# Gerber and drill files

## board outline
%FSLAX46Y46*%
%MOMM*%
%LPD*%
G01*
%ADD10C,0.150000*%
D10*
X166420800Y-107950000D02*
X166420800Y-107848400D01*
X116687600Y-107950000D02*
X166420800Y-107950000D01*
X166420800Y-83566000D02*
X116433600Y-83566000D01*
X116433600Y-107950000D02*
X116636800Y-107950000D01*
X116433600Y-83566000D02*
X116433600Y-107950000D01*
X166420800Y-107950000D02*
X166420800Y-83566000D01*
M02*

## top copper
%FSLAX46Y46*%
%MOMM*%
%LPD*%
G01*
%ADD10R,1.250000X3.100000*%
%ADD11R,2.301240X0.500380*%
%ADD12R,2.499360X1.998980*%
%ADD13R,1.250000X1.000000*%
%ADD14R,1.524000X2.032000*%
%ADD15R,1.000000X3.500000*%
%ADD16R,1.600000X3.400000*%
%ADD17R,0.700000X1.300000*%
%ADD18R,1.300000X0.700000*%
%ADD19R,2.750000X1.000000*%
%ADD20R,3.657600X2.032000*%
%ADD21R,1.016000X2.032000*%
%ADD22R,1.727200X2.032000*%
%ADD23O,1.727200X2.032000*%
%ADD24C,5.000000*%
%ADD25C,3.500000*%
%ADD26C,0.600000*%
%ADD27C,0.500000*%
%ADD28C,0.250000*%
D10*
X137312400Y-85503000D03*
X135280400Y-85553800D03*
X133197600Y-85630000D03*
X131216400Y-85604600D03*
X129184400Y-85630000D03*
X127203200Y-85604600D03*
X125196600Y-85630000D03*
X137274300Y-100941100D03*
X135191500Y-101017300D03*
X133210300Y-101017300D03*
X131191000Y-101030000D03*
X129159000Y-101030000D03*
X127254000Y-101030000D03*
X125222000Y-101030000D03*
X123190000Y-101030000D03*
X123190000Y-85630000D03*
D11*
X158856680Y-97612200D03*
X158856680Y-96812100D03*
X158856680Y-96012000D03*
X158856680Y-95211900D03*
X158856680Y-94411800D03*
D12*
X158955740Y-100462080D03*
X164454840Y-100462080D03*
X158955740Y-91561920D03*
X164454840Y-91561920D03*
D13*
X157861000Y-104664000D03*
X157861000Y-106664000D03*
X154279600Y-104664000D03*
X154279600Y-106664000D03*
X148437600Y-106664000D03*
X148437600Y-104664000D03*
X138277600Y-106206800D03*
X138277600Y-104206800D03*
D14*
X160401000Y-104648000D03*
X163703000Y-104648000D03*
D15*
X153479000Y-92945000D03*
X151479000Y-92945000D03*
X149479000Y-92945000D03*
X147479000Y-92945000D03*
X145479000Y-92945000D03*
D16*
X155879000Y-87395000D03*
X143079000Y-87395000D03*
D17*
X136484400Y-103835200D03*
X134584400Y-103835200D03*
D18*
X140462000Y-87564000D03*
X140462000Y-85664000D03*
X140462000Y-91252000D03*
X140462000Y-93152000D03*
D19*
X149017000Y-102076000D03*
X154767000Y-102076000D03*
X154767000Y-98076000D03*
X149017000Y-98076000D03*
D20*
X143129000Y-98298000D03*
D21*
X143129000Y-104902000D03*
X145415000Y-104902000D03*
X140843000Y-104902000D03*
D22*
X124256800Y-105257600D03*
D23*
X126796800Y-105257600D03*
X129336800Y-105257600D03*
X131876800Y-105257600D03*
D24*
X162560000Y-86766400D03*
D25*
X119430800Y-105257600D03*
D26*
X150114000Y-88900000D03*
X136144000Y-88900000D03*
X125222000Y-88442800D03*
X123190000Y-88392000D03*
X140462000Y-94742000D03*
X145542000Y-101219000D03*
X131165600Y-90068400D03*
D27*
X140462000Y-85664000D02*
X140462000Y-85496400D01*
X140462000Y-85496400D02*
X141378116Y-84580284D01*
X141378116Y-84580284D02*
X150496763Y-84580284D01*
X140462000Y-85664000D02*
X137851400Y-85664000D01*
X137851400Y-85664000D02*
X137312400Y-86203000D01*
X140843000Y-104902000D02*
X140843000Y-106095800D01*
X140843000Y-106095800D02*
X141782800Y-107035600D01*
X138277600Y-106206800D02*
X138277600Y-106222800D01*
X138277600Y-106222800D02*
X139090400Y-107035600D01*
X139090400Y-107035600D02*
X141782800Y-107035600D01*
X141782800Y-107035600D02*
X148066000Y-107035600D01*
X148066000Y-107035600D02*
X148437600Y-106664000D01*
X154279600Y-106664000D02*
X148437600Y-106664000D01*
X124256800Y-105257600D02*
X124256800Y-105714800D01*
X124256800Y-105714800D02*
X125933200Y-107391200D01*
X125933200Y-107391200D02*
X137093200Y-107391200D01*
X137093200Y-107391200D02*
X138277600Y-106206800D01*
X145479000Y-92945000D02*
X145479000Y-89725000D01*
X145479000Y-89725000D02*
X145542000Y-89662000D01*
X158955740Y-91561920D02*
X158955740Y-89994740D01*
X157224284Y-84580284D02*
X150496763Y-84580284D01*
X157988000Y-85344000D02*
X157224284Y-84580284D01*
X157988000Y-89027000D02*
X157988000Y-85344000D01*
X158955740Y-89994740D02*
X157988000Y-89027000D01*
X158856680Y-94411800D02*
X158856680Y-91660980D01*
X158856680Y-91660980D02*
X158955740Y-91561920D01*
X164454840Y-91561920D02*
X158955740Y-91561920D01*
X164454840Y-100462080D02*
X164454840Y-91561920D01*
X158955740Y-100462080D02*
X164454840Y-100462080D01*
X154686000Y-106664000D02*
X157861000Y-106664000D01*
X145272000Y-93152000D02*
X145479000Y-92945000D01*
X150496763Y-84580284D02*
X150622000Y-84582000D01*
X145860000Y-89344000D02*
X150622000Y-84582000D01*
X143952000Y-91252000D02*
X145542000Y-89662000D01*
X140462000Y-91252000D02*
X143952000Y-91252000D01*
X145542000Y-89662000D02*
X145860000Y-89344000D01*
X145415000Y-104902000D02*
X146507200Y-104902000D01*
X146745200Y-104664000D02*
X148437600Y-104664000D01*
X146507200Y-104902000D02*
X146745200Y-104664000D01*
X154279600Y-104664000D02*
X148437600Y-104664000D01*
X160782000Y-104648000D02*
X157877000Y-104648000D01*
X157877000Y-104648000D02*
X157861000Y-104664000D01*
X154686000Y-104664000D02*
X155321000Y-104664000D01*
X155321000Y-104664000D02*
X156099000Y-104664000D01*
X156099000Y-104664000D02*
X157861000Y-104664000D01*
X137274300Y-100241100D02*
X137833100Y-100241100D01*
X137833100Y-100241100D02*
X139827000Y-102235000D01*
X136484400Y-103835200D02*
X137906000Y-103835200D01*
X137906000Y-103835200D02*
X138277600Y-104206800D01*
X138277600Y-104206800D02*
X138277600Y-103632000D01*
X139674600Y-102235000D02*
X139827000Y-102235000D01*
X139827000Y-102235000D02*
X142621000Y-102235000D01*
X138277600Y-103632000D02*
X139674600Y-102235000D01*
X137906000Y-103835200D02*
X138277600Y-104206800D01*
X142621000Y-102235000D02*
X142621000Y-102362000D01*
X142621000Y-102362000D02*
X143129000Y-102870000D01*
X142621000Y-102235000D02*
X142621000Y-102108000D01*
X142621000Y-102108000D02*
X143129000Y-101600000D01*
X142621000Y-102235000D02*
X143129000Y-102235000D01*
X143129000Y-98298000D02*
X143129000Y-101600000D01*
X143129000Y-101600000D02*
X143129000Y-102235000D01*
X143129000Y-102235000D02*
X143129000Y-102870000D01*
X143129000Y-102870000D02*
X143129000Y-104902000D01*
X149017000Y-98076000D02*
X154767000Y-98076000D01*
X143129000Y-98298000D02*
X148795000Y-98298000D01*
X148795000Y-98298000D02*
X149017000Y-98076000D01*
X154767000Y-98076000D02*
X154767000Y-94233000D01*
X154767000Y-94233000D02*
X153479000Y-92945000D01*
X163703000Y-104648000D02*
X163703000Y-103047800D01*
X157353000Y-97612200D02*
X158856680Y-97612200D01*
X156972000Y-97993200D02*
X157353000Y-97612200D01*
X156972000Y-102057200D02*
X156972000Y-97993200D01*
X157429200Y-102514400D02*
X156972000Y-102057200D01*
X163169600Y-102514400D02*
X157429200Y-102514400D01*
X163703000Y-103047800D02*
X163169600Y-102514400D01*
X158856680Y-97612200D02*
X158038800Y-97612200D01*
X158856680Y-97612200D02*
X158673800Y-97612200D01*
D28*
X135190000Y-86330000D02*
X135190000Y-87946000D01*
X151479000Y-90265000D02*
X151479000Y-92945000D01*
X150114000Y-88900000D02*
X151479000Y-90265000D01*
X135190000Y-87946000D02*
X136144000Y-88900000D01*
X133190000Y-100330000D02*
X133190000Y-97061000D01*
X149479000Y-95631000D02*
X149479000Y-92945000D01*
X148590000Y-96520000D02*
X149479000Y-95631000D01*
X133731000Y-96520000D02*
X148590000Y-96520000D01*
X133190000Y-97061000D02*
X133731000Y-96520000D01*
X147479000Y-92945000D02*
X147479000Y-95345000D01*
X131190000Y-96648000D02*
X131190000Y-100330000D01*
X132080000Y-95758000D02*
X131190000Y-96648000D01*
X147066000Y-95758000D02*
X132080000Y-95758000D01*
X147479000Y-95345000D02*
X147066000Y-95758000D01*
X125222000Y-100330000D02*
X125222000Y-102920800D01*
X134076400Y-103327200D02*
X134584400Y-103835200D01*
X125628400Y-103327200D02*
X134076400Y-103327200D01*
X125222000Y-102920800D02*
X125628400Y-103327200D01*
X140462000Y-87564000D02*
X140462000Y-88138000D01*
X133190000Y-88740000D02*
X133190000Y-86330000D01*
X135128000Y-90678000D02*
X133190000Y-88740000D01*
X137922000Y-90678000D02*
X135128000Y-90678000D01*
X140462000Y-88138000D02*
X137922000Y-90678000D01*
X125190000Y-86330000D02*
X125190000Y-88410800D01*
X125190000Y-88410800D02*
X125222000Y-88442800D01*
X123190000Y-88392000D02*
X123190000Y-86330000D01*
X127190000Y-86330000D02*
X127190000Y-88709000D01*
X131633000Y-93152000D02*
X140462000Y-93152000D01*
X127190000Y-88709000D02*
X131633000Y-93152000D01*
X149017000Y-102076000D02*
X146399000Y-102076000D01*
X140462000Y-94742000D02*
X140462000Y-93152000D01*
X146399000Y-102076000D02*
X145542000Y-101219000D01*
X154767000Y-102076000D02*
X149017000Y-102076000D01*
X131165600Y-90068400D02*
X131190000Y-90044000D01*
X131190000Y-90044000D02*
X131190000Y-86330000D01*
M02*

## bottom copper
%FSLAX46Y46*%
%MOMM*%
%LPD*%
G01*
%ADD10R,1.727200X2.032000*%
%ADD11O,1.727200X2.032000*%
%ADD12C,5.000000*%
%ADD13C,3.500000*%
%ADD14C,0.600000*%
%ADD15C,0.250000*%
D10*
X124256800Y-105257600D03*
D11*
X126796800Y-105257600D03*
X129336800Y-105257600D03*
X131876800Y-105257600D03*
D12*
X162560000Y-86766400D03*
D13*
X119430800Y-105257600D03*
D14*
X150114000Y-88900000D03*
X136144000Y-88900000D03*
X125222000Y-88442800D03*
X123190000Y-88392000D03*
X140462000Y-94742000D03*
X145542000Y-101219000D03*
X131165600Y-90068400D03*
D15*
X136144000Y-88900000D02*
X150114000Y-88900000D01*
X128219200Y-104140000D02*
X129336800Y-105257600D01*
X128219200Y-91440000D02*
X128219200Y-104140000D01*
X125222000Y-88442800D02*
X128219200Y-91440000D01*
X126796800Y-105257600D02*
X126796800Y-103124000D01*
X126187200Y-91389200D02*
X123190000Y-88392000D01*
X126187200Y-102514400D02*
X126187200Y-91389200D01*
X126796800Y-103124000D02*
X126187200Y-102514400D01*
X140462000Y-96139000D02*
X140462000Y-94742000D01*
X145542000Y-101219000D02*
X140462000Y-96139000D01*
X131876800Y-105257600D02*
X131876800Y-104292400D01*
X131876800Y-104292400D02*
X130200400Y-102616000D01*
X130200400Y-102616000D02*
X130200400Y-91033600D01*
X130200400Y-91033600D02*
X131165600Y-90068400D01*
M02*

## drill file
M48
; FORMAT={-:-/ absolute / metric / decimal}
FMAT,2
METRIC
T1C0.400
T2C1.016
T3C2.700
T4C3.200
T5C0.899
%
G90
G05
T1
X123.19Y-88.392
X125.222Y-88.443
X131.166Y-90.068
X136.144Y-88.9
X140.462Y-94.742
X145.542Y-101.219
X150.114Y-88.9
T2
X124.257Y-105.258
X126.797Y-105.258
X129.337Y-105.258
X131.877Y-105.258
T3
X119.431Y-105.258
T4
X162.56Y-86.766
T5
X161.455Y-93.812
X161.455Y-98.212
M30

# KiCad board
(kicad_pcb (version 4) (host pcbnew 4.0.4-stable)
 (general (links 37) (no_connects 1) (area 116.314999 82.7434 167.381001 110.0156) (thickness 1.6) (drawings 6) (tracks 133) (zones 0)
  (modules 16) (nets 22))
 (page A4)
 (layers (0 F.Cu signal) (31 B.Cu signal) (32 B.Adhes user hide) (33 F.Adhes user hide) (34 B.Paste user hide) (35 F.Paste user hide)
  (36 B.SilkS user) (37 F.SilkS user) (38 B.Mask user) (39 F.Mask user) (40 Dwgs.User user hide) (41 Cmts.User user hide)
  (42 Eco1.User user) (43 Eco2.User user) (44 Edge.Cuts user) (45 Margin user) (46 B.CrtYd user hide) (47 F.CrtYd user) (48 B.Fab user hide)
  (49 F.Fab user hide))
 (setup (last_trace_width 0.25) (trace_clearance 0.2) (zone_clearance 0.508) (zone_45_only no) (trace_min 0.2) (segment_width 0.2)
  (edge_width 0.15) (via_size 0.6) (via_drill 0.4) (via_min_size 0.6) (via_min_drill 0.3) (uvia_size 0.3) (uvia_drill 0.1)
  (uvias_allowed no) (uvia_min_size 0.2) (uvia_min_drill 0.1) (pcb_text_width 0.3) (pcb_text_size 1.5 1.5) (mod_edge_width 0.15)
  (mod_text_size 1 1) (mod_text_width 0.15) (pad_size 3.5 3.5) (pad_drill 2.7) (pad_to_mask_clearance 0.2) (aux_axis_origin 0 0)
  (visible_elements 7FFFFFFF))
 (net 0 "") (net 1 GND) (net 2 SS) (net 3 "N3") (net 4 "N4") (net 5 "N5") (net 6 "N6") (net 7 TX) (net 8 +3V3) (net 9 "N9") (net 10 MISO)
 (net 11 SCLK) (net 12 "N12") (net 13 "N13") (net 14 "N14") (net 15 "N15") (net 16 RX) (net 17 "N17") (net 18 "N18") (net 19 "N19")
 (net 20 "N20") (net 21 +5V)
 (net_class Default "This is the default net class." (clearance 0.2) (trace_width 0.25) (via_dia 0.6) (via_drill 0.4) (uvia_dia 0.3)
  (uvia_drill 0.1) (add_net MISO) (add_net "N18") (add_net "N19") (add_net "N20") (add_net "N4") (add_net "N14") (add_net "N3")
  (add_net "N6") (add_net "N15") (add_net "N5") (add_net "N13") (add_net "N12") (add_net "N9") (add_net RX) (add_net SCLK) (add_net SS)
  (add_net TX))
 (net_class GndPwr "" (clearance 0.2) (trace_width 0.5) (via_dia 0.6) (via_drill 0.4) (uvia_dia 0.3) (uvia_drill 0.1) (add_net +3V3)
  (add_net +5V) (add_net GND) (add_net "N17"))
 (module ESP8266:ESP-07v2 (layer F.Cu) (at 123.19 100.33 90)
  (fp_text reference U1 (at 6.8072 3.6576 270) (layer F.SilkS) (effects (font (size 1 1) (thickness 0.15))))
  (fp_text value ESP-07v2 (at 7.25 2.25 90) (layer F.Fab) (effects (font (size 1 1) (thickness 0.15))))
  (pad 9 smd rect (at 14.127 14.1224 90) (size 3.1 1.25) (drill (offset 0.7 0)) (layers F.Cu F.Paste F.Mask) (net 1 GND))
  (pad 10 smd rect (at 14.0762 12.0904 90) (size 3.1 1.25) (drill (offset 0.7 0)) (layers F.Cu F.Paste F.Mask) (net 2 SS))
  (pad 11 smd rect (at 14 10.0076 90) (size 3.1 1.25) (drill (offset 0.7 0)) (layers F.Cu F.Paste F.Mask) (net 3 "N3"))
  (pad 12 smd rect (at 14.0254 8.0264 90) (size 3.1 1.25) (drill (offset 0.7 0)) (layers F.Cu F.Paste F.Mask) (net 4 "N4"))
  (pad 13 smd rect (at 14 5.9944 90) (size 3.1 1.25) (drill (offset 0.7 0)) (layers F.Cu F.Paste F.Mask) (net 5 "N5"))
  (pad 14 smd rect (at 14.0254 4.0132 90) (size 3.1 1.25) (drill (offset 0.7 0)) (layers F.Cu F.Paste F.Mask) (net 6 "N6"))
  (pad 15 smd rect (at 14 2.0066 90) (size 3.1 1.25) (drill (offset 0.7 0)) (layers F.Cu F.Paste F.Mask) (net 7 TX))
  (pad 8 smd rect (at 0.0889 14.0843 90) (size 3.1 1.25) (drill (offset -0.7 0)) (layers F.Cu F.Paste F.Mask) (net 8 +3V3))
  (pad 7 smd rect (at 0.0127 12.0015 90) (size 3.1 1.25) (drill (offset -0.7 0)) (layers F.Cu F.Paste F.Mask) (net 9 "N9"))
  (pad 6 smd rect (at 0.0127 10.0203 90) (size 3.1 1.25) (drill (offset -0.7 0)) (layers F.Cu F.Paste F.Mask) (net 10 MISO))
  (pad 5 smd rect (at 0 8.001 90) (size 3.1 1.25) (drill (offset -0.7 0)) (layers F.Cu F.Paste F.Mask) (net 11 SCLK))
  (pad 4 smd rect (at 0 5.969 90) (size 3.1 1.25) (drill (offset -0.7 0)) (layers F.Cu F.Paste F.Mask) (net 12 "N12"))
  (pad 3 smd rect (at 0 4.064 90) (size 3.1 1.25) (drill (offset -0.7 0)) (layers F.Cu F.Paste F.Mask) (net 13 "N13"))
  (pad 2 smd rect (at 0 2.032 90) (size 3.1 1.25) (drill (offset -0.7 0)) (layers F.Cu F.Paste F.Mask) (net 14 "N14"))
  (pad 1 smd rect (at 0 0 90) (size 3.1 1.25) (drill (offset -0.7 0)) (layers F.Cu F.Paste F.Mask) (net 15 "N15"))
  (pad 16 smd rect (at 14 0 90) (size 3.1 1.25) (drill (offset 0.7 0)) (layers F.Cu F.Paste F.Mask) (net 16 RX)))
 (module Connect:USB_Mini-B (layer F.Cu) (at 162.306 96.012 180)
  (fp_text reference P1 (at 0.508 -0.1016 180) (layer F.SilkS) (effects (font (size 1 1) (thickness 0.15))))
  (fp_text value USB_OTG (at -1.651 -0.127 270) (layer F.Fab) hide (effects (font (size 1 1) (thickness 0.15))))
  (pad 1 smd rect (at 3.44932 -1.6002 180) (size 2.30124 0.50038) (layers F.Cu F.Paste F.Mask) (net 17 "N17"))
  (pad 2 smd rect (at 3.44932 -0.8001 180) (size 2.30124 0.50038) (layers F.Cu F.Paste F.Mask) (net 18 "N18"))
  (pad 3 smd rect (at 3.44932 0 180) (size 2.30124 0.50038) (layers F.Cu F.Paste F.Mask) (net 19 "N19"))
  (pad 4 smd rect (at 3.44932 0.8001 180) (size 2.30124 0.50038) (layers F.Cu F.Paste F.Mask) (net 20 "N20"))
  (pad 5 smd rect (at 3.44932 1.6002 180) (size 2.30124 0.50038) (layers F.Cu F.Paste F.Mask) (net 1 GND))
  (pad 6 smd rect (at 3.35026 -4.45008 180) (size 2.49936 1.99898) (layers F.Cu F.Paste F.Mask) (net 1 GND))
  (pad 6 smd rect (at -2.14884 -4.45008 180) (size 2.49936 1.99898) (layers F.Cu F.Paste F.Mask) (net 1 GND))
  (pad 6 smd rect (at 3.35026 4.45008 180) (size 2.49936 1.99898) (layers F.Cu F.Paste F.Mask) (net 1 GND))
  (pad 6 smd rect (at -2.14884 4.45008 180) (size 2.49936 1.99898) (layers F.Cu F.Paste F.Mask) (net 1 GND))
  (pad "" np_thru_hole circle (at 0.8509 -2.19964 180) (size 0.89916 0.89916) (drill 0.89916) (layers *.Cu *.Mask F.SilkS))
  (pad "" np_thru_hole circle (at 0.8509 2.19964 180) (size 0.89916 0.89916) (drill 0.89916) (layers *.Cu *.Mask F.SilkS)))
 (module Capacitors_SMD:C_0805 (layer F.Cu) (at 157.861 105.664 270)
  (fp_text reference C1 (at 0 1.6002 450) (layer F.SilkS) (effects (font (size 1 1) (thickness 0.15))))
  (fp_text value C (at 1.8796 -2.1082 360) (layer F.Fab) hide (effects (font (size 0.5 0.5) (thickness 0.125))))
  (pad 1 smd rect (at -1 0 270) (size 1 1.25) (layers F.Cu F.Paste F.Mask) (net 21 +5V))
  (pad 2 smd rect (at 1 0 270) (size 1 1.25) (layers F.Cu F.Paste F.Mask) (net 1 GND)))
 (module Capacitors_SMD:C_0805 (layer F.Cu) (at 154.2796 105.664 270)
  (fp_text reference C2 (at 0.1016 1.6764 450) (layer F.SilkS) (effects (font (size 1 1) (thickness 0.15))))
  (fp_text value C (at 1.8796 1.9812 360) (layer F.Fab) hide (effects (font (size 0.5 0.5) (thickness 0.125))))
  (pad 1 smd rect (at -1 0 270) (size 1 1.25) (layers F.Cu F.Paste F.Mask) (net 21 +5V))
  (pad 2 smd rect (at 1 0 270) (size 1 1.25) (layers F.Cu F.Paste F.Mask) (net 1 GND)))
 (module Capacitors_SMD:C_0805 (layer F.Cu) (at 148.4376 105.664 90)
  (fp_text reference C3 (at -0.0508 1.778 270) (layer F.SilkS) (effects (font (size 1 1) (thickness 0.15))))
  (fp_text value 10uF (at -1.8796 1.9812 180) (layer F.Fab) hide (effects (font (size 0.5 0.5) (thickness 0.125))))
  (pad 1 smd rect (at -1 0 90) (size 1 1.25) (layers F.Cu F.Paste F.Mask) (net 1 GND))
  (pad 2 smd rect (at 1 0 90) (size 1 1.25) (layers F.Cu F.Paste F.Mask) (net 21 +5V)))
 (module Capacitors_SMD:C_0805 (layer F.Cu) (at 138.2776 105.2068 90)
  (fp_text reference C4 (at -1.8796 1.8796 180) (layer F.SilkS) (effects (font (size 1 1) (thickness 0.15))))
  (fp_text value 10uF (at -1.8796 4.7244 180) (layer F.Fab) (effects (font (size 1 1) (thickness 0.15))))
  (pad 1 smd rect (at -1 0 90) (size 1 1.25) (layers F.Cu F.Paste F.Mask) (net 1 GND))
  (pad 2 smd rect (at 1 0 90) (size 1 1.25) (layers F.Cu F.Paste F.Mask) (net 8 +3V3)))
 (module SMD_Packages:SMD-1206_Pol (layer F.Cu) (at 162.052 104.648)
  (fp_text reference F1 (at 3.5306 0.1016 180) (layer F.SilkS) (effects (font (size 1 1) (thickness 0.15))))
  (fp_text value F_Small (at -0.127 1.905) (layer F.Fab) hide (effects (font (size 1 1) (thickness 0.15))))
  (pad 1 smd rect (at -1.651 0) (size 1.524 2.032) (layers F.Cu F.Paste F.Mask) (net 21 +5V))
  (pad 2 smd rect (at 1.651 0) (size 1.524 2.032) (layers F.Cu F.Paste F.Mask) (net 17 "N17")))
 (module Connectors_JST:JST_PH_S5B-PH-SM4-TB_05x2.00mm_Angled (layer F.Cu) (at 149.479 90.17 180)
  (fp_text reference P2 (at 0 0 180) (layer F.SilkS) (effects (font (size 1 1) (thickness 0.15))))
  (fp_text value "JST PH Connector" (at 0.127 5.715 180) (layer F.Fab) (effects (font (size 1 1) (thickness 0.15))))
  (pad 1 smd rect (at -4 -2.775 180) (size 1 3.5) (layers F.Cu F.Paste F.Mask) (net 8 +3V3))
  (pad 2 smd rect (at -2 -2.775 180) (size 1 3.5) (layers F.Cu F.Paste F.Mask) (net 2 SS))
  (pad 3 smd rect (at 0 -2.775 180) (size 1 3.5) (layers F.Cu F.Paste F.Mask) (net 10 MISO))
  (pad 4 smd rect (at 2 -2.775 180) (size 1 3.5) (layers F.Cu F.Paste F.Mask) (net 11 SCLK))
  (pad 5 smd rect (at 4 -2.775 180) (size 1 3.5) (layers F.Cu F.Paste F.Mask) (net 1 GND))
  (pad "" smd rect (at -6.4 2.775 180) (size 1.6 3.4) (layers F.Cu F.Paste F.Mask))
  (pad "" smd rect (at 6.4 2.775 180) (size 1.6 3.4) (layers F.Cu F.Paste F.Mask)))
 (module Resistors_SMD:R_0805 (layer F.Cu) (at 135.5344 103.8352 180)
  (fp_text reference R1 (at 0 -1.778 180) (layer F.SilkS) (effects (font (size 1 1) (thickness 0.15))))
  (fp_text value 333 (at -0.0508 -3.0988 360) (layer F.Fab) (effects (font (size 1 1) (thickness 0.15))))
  (pad 1 smd rect (at -0.95 0 180) (size 0.7 1.3) (layers F.Cu F.Paste F.Mask) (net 8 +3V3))
  (pad 2 smd rect (at 0.95 0 180) (size 0.7 1.3) (layers F.Cu F.Paste F.Mask) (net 14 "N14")))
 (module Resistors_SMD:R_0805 (layer F.Cu) (at 140.462 86.614 90)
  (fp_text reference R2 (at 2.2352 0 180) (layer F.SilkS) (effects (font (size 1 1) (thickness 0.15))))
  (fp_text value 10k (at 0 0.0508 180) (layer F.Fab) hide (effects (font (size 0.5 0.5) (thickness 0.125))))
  (pad 1 smd rect (at -0.95 0 90) (size 0.7 1.3) (layers F.Cu F.Paste F.Mask) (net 3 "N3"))
  (pad 2 smd rect (at 0.95 0 90) (size 0.7 1.3) (layers F.Cu F.Paste F.Mask) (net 1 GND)))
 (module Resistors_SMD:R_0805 (layer F.Cu) (at 140.462 92.202 270)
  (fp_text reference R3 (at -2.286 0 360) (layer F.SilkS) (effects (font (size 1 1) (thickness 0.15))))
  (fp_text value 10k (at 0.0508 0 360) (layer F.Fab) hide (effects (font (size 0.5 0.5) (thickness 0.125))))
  (pad 1 smd rect (at -0.95 0 270) (size 0.7 1.3) (layers F.Cu F.Paste F.Mask) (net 1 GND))
  (pad 2 smd rect (at 0.95 0 270) (size 0.7 1.3) (layers F.Cu F.Paste F.Mask) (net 6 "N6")))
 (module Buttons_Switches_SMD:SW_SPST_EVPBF (layer F.Cu) (at 151.892 100.076 180)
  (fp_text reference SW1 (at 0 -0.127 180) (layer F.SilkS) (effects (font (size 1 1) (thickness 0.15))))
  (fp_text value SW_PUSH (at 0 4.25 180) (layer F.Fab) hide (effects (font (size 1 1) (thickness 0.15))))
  (pad 1 smd rect (at 2.875 -2 180) (size 2.75 1) (layers F.Cu F.Paste F.Mask) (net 6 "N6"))
  (pad 1 smd rect (at -2.875 -2 180) (size 2.75 1) (layers F.Cu F.Paste F.Mask) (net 6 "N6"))
  (pad 2 smd rect (at -2.875 2 180) (size 2.75 1) (layers F.Cu F.Paste F.Mask) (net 8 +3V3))
  (pad 2 smd rect (at 2.875 2 180) (size 2.75 1) (layers F.Cu F.Paste F.Mask) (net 8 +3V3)))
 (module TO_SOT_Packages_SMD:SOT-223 (layer F.Cu) (at 143.129 101.6)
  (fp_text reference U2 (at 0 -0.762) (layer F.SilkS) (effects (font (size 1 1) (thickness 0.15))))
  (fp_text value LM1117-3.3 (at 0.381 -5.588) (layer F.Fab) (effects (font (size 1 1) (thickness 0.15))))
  (pad 4 smd rect (at 0 -3.302) (size 3.6576 2.032) (layers F.Cu F.Paste F.Mask) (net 8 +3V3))
  (pad 2 smd rect (at 0 3.302) (size 1.016 2.032) (layers F.Cu F.Paste F.Mask) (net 8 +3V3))
  (pad 3 smd rect (at 2.286 3.302) (size 1.016 2.032) (layers F.Cu F.Paste F.Mask) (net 21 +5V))
  (pad 1 smd rect (at -2.286 3.302) (size 1.016 2.032) (layers F.Cu F.Paste F.Mask) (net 1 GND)))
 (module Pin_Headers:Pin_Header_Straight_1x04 (layer F.Cu) (at 124.2568 105.2576 90)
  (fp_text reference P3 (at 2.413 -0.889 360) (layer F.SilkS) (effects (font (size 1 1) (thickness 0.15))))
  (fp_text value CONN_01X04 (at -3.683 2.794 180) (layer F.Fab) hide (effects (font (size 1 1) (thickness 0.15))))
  (pad 1 thru_hole rect (at 0 0 90) (size 2.032 1.7272) (drill 1.016) (layers *.Cu *.Mask F.SilkS) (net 1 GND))
  (pad 2 thru_hole oval (at 0 2.54 90) (size 2.032 1.7272) (drill 1.016) (layers *.Cu *.Mask F.SilkS) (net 16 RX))
  (pad 3 thru_hole oval (at 0 5.08 90) (size 2.032 1.7272) (drill 1.016) (layers *.Cu *.Mask F.SilkS) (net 7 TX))
  (pad 4 thru_hole oval (at 0 7.62 90) (size 2.032 1.7272) (drill 1.016) (layers *.Cu *.Mask F.SilkS) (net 4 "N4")))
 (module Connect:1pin (layer F.Cu) (at 162.56 86.7664)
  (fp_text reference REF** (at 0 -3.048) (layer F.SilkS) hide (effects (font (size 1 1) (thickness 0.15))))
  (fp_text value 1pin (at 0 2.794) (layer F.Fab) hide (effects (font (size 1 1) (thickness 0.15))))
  (pad 1 thru_hole circle (at 0 0) (size 5 5) (drill 3.2) (layers *.Cu *.Mask F.SilkS)))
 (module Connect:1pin (layer F.Cu) (at 119.4308 105.2576)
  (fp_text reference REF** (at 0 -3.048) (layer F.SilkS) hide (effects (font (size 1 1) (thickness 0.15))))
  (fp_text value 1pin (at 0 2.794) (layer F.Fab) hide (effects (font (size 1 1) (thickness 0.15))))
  (pad 1 thru_hole circle (at 0 0) (size 3.5 3.5) (drill 2.7) (layers *.Cu *.Mask F.SilkS)))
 (gr_line (start 166.4208 107.95) (end 166.4208 107.8484) (angle 90) (layer Edge.Cuts) (width 0.15))
 (gr_line (start 116.6876 107.95) (end 166.4208 107.95) (angle 90) (layer Edge.Cuts) (width 0.15))
 (gr_line (start 166.4208 83.566) (end 116.4336 83.566) (angle 90) (layer Edge.Cuts) (width 0.15))
 (gr_line (start 116.4336 107.95) (end 116.6368 107.95) (angle 90) (layer Edge.Cuts) (width 0.15))
 (gr_line (start 116.4336 83.566) (end 116.4336 107.95) (angle 90) (layer Edge.Cuts) (width 0.15))
 (gr_line (start 166.4208 107.95) (end 166.4208 83.566) (angle 90) (layer Edge.Cuts) (width 0.15))
 (segment (start 140.462 85.664) (end 140.462 85.4964) (width 0.5) (layer F.Cu) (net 1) (status C00000))
 (segment (start 140.462 85.4964) (end 141.378116 84.580284) (width 0.5) (layer F.Cu) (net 1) (status 400000))
 (segment (start 141.378116 84.580284) (end 150.496763 84.580284) (width 0.5) (layer F.Cu) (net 1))
 (segment (start 140.462 85.664) (end 137.8514 85.664) (width 0.5) (layer F.Cu) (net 1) (status C00000))
 (segment (start 137.8514 85.664) (end 137.3124 86.203) (width 0.5) (layer F.Cu) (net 1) (status C00000))
 (segment (start 140.843 104.902) (end 140.843 106.0958) (width 0.5) (layer F.Cu) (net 1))
 (segment (start 140.843 106.0958) (end 141.7828 107.0356) (width 0.5) (layer F.Cu) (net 1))
 (segment (start 138.2776 106.2068) (end 138.2776 106.2228) (width 0.5) (layer F.Cu) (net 1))
 (segment (start 138.2776 106.2228) (end 139.0904 107.0356) (width 0.5) (layer F.Cu) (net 1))
 (segment (start 139.0904 107.0356) (end 141.7828 107.0356) (width 0.5) (layer F.Cu) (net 1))
 (segment (start 141.7828 107.0356) (end 148.066 107.0356) (width 0.5) (layer F.Cu) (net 1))
 (segment (start 148.066 107.0356) (end 148.4376 106.664) (width 0.5) (layer F.Cu) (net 1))
 (segment (start 154.2796 106.664) (end 148.4376 106.664) (width 0.5) (layer F.Cu) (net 1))
 (segment (start 124.2568 105.2576) (end 124.2568 105.7148) (width 0.5) (layer F.Cu) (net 1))
 (segment (start 124.2568 105.7148) (end 125.9332 107.3912) (width 0.5) (layer F.Cu) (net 1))
 (segment (start 125.9332 107.3912) (end 137.0932 107.3912) (width 0.5) (layer F.Cu) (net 1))
 (segment (start 137.0932 107.3912) (end 138.2776 106.2068) (width 0.5) (layer F.Cu) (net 1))
 (segment (start 145.479 92.945) (end 145.479 89.725) (width 0.5) (layer F.Cu) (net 1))
 (segment (start 145.479 89.725) (end 145.542 89.662) (width 0.5) (layer F.Cu) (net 1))
 (segment (start 158.95574 91.56192) (end 158.95574 89.99474) (width 0.5) (layer F.Cu) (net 1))
 (segment (start 157.224284 84.580284) (end 150.496763 84.580284) (width 0.5) (layer F.Cu) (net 1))
 (segment (start 157.988 85.344) (end 157.224284 84.580284) (width 0.5) (layer F.Cu) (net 1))
 (segment (start 157.988 89.027) (end 157.988 85.344) (width 0.5) (layer F.Cu) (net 1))
 (segment (start 158.95574 89.99474) (end 157.988 89.027) (width 0.5) (layer F.Cu) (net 1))
 (segment (start 158.85668 94.4118) (end 158.85668 91.66098) (width 0.5) (layer F.Cu) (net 1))
 (segment (start 158.85668 91.66098) (end 158.95574 91.56192) (width 0.5) (layer F.Cu) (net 1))
 (segment (start 164.45484 91.56192) (end 158.95574 91.56192) (width 0.5) (layer F.Cu) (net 1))
 (segment (start 164.45484 100.46208) (end 164.45484 91.56192) (width 0.5) (layer F.Cu) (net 1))
 (segment (start 158.95574 100.46208) (end 164.45484 100.46208) (width 0.5) (layer F.Cu) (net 1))
 (segment (start 154.686 106.664) (end 157.861 106.664) (width 0.5) (layer F.Cu) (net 1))
 (segment (start 145.272 93.152) (end 145.479 92.945) (width 0.5) (layer F.Cu) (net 1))
 (segment (start 150.496763 84.580284) (end 150.622 84.582) (width 0.5) (layer F.Cu) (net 1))
 (segment (start 145.86 89.344) (end 150.622 84.582) (width 0.5) (layer F.Cu) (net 1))
 (segment (start 143.952 91.252) (end 145.542 89.662) (width 0.5) (layer F.Cu) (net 1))
 (segment (start 140.462 91.252) (end 143.952 91.252) (width 0.5) (layer F.Cu) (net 1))
 (segment (start 145.542 89.662) (end 145.86 89.344) (width 0.5) (layer F.Cu) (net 1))
 (segment (start 145.415 104.902) (end 146.5072 104.902) (width 0.5) (layer F.Cu) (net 21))
 (segment (start 146.7452 104.664) (end 148.4376 104.664) (width 0.5) (layer F.Cu) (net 21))
 (segment (start 146.5072 104.902) (end 146.7452 104.664) (width 0.5) (layer F.Cu) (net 21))
 (segment (start 154.2796 104.664) (end 148.4376 104.664) (width 0.5) (layer F.Cu) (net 21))
 (segment (start 160.782 104.648) (end 157.877 104.648) (width 0.5) (layer F.Cu) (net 21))
 (segment (start 157.877 104.648) (end 157.861 104.664) (width 0.5) (layer F.Cu) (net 21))
 (segment (start 154.686 104.664) (end 155.321 104.664) (width 0.5) (layer F.Cu) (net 21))
 (segment (start 155.321 104.664) (end 156.099 104.664) (width 0.5) (layer F.Cu) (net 21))
 (segment (start 156.099 104.664) (end 157.861 104.664) (width 0.5) (layer F.Cu) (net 21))
 (segment (start 137.2743 100.2411) (end 137.8331 100.2411) (width 0.5) (layer F.Cu) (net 8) (status C00000))
 (segment (start 137.8331 100.2411) (end 139.827 102.235) (width 0.5) (layer F.Cu) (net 8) (status 400000))
 (segment (start 136.4844 103.8352) (end 137.906 103.8352) (width 0.5) (layer F.Cu) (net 8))
 (segment (start 137.906 103.8352) (end 138.2776 104.2068) (width 0.5) (layer F.Cu) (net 8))
 (segment (start 138.2776 104.2068) (end 138.2776 103.632) (width 0.5) (layer F.Cu) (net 8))
 (segment (start 139.6746 102.235) (end 139.827 102.235) (width 0.5) (layer F.Cu) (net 8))
 (segment (start 139.827 102.235) (end 142.621 102.235) (width 0.5) (layer F.Cu) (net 8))
 (segment (start 138.2776 103.632) (end 139.6746 102.235) (width 0.5) (layer F.Cu) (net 8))
 (segment (start 137.906 103.8352) (end 138.2776 104.2068) (width 0.5) (layer F.Cu) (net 8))
 (segment (start 142.621 102.235) (end 142.621 102.362) (width 0.5) (layer F.Cu) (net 8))
 (segment (start 142.621 102.362) (end 143.129 102.87) (width 0.5) (layer F.Cu) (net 8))
 (segment (start 142.621 102.235) (end 142.621 102.108) (width 0.5) (layer F.Cu) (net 8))
 (segment (start 142.621 102.108) (end 143.129 101.6) (width 0.5) (layer F.Cu) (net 8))
 (segment (start 142.621 102.235) (end 143.129 102.235) (width 0.5) (layer F.Cu) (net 8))
 (segment (start 143.129 98.298) (end 143.129 101.6) (width 0.5) (layer F.Cu) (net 8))
 (segment (start 143.129 101.6) (end 143.129 102.235) (width 0.5) (layer F.Cu) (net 8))
 (segment (start 143.129 102.235) (end 143.129 102.87) (width 0.5) (layer F.Cu) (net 8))
 (segment (start 143.129 102.87) (end 143.129 104.902) (width 0.5) (layer F.Cu) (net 8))
 (segment (start 149.017 98.076) (end 154.767 98.076) (width 0.5) (layer F.Cu) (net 8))
 (segment (start 143.129 98.298) (end 148.795 98.298) (width 0.5) (layer F.Cu) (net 8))
 (segment (start 148.795 98.298) (end 149.017 98.076) (width 0.5) (layer F.Cu) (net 8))
 (segment (start 154.767 98.076) (end 154.767 94.233) (width 0.5) (layer F.Cu) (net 8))
 (segment (start 154.767 94.233) (end 153.479 92.945) (width 0.5) (layer F.Cu) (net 8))
 (segment (start 163.703 104.648) (end 163.703 103.0478) (width 0.5) (layer F.Cu) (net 17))
 (segment (start 157.353 97.6122) (end 158.85668 97.6122) (width 0.5) (layer F.Cu) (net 17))
 (segment (start 156.972 97.9932) (end 157.353 97.6122) (width 0.5) (layer F.Cu) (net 17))
 (segment (start 156.972 102.0572) (end 156.972 97.9932) (width 0.5) (layer F.Cu) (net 17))
 (segment (start 157.4292 102.5144) (end 156.972 102.0572) (width 0.5) (layer F.Cu) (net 17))
 (segment (start 163.1696 102.5144) (end 157.4292 102.5144) (width 0.5) (layer F.Cu) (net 17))
 (segment (start 163.703 103.0478) (end 163.1696 102.5144) (width 0.5) (layer F.Cu) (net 17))
 (segment (start 158.85668 97.6122) (end 158.0388 97.6122) (width 0.5) (layer F.Cu) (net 17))
 (segment (start 158.85668 97.6122) (end 158.6738 97.6122) (width 0.5) (layer F.Cu) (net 17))
 (segment (start 135.19 86.33) (end 135.19 87.946) (width 0.25) (layer F.Cu) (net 2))
 (segment (start 151.479 90.265) (end 151.479 92.945) (width 0.25) (layer F.Cu) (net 2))
 (segment (start 150.114 88.9) (end 151.479 90.265) (width 0.25) (layer F.Cu) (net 2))
 (via (at 150.114 88.9) (size 0.6) (drill 0.4) (layers F.Cu B.Cu) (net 2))
 (segment (start 136.144 88.9) (end 150.114 88.9) (width 0.25) (layer B.Cu) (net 2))
 (via (at 136.144 88.9) (size 0.6) (drill 0.4) (layers F.Cu B.Cu) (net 2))
 (segment (start 135.19 87.946) (end 136.144 88.9) (width 0.25) (layer F.Cu) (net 2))
 (segment (start 133.19 100.33) (end 133.19 97.061) (width 0.25) (layer F.Cu) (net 10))
 (segment (start 149.479 95.631) (end 149.479 92.945) (width 0.25) (layer F.Cu) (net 10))
 (segment (start 148.59 96.52) (end 149.479 95.631) (width 0.25) (layer F.Cu) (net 10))
 (segment (start 133.731 96.52) (end 148.59 96.52) (width 0.25) (layer F.Cu) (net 10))
 (segment (start 133.19 97.061) (end 133.731 96.52) (width 0.25) (layer F.Cu) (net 10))
 (segment (start 147.479 92.945) (end 147.479 95.345) (width 0.25) (layer F.Cu) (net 11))
 (segment (start 131.19 96.648) (end 131.19 100.33) (width 0.25) (layer F.Cu) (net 11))
 (segment (start 132.08 95.758) (end 131.19 96.648) (width 0.25) (layer F.Cu) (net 11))
 (segment (start 147.066 95.758) (end 132.08 95.758) (width 0.25) (layer F.Cu) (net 11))
 (segment (start 147.479 95.345) (end 147.066 95.758) (width 0.25) (layer F.Cu) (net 11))
 (segment (start 125.222 100.33) (end 125.222 102.9208) (width 0.25) (layer F.Cu) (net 14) (status 400000))
 (segment (start 134.0764 103.3272) (end 134.5844 103.8352) (width 0.25) (layer F.Cu) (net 14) (status 800000))
 (segment (start 125.6284 103.3272) (end 134.0764 103.3272) (width 0.25) (layer F.Cu) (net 14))
 (segment (start 125.222 102.9208) (end 125.6284 103.3272) (width 0.25) (layer F.Cu) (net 14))
 (segment (start 140.462 87.564) (end 140.462 88.138) (width 0.25) (layer F.Cu) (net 3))
 (segment (start 133.19 88.74) (end 133.19 86.33) (width 0.25) (layer F.Cu) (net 3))
 (segment (start 135.128 90.678) (end 133.19 88.74) (width 0.25) (layer F.Cu) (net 3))
 (segment (start 137.922 90.678) (end 135.128 90.678) (width 0.25) (layer F.Cu) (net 3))
 (segment (start 140.462 88.138) (end 137.922 90.678) (width 0.25) (layer F.Cu) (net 3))
 (segment (start 125.19 86.33) (end 125.19 88.4108) (width 0.25) (layer F.Cu) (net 7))
 (segment (start 128.2192 104.14) (end 129.3368 105.2576) (width 0.25) (layer B.Cu) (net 7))
 (segment (start 128.2192 91.44) (end 128.2192 104.14) (width 0.25) (layer B.Cu) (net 7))
 (segment (start 125.222 88.4428) (end 128.2192 91.44) (width 0.25) (layer B.Cu) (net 7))
 (via (at 125.222 88.4428) (size 0.6) (drill 0.4) (layers F.Cu B.Cu) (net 7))
 (segment (start 125.19 88.4108) (end 125.222 88.4428) (width 0.25) (layer F.Cu) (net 7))
 (segment (start 126.7968 105.2576) (end 126.7968 103.124) (width 0.25) (layer B.Cu) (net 16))
 (segment (start 123.19 88.392) (end 123.19 86.33) (width 0.25) (layer F.Cu) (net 16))
 (via (at 123.19 88.392) (size 0.6) (drill 0.4) (layers F.Cu B.Cu) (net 16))
 (segment (start 126.1872 91.3892) (end 123.19 88.392) (width 0.25) (layer B.Cu) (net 16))
 (segment (start 126.1872 102.5144) (end 126.1872 91.3892) (width 0.25) (layer B.Cu) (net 16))
 (segment (start 126.7968 103.124) (end 126.1872 102.5144) (width 0.25) (layer B.Cu) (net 16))
 (segment (start 127.19 86.33) (end 127.19 88.709) (width 0.25) (layer F.Cu) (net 6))
 (segment (start 131.633 93.152) (end 140.462 93.152) (width 0.25) (layer F.Cu) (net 6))
 (segment (start 127.19 88.709) (end 131.633 93.152) (width 0.25) (layer F.Cu) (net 6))
 (segment (start 149.017 102.076) (end 146.399 102.076) (width 0.25) (layer F.Cu) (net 6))
 (segment (start 140.462 94.742) (end 140.462 93.152) (width 0.25) (layer F.Cu) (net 6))
 (via (at 140.462 94.742) (size 0.6) (drill 0.4) (layers F.Cu B.Cu) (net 6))
 (segment (start 140.462 96.139) (end 140.462 94.742) (width 0.25) (layer B.Cu) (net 6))
 (segment (start 145.542 101.219) (end 140.462 96.139) (width 0.25) (layer B.Cu) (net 6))
 (via (at 145.542 101.219) (size 0.6) (drill 0.4) (layers F.Cu B.Cu) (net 6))
 (segment (start 146.399 102.076) (end 145.542 101.219) (width 0.25) (layer F.Cu) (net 6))
 (segment (start 154.767 102.076) (end 149.017 102.076) (width 0.25) (layer F.Cu) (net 6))
 (segment (start 131.8768 105.2576) (end 131.8768 104.2924) (width 0.25) (layer B.Cu) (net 4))
 (segment (start 131.8768 104.2924) (end 130.2004 102.616) (width 0.25) (layer B.Cu) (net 4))
 (segment (start 130.2004 102.616) (end 130.2004 91.0336) (width 0.25) (layer B.Cu) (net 4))
 (segment (start 130.2004 91.0336) (end 131.1656 90.0684) (width 0.25) (layer B.Cu) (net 4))
 (via (at 131.1656 90.0684) (size 0.6) (drill 0.4) (layers F.Cu B.Cu) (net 4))
 (segment (start 131.1656 90.0684) (end 131.19 90.044) (width 0.25) (layer F.Cu) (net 4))
 (segment (start 131.19 90.044) (end 131.19 86.33) (width 0.25) (layer F.Cu) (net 4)))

